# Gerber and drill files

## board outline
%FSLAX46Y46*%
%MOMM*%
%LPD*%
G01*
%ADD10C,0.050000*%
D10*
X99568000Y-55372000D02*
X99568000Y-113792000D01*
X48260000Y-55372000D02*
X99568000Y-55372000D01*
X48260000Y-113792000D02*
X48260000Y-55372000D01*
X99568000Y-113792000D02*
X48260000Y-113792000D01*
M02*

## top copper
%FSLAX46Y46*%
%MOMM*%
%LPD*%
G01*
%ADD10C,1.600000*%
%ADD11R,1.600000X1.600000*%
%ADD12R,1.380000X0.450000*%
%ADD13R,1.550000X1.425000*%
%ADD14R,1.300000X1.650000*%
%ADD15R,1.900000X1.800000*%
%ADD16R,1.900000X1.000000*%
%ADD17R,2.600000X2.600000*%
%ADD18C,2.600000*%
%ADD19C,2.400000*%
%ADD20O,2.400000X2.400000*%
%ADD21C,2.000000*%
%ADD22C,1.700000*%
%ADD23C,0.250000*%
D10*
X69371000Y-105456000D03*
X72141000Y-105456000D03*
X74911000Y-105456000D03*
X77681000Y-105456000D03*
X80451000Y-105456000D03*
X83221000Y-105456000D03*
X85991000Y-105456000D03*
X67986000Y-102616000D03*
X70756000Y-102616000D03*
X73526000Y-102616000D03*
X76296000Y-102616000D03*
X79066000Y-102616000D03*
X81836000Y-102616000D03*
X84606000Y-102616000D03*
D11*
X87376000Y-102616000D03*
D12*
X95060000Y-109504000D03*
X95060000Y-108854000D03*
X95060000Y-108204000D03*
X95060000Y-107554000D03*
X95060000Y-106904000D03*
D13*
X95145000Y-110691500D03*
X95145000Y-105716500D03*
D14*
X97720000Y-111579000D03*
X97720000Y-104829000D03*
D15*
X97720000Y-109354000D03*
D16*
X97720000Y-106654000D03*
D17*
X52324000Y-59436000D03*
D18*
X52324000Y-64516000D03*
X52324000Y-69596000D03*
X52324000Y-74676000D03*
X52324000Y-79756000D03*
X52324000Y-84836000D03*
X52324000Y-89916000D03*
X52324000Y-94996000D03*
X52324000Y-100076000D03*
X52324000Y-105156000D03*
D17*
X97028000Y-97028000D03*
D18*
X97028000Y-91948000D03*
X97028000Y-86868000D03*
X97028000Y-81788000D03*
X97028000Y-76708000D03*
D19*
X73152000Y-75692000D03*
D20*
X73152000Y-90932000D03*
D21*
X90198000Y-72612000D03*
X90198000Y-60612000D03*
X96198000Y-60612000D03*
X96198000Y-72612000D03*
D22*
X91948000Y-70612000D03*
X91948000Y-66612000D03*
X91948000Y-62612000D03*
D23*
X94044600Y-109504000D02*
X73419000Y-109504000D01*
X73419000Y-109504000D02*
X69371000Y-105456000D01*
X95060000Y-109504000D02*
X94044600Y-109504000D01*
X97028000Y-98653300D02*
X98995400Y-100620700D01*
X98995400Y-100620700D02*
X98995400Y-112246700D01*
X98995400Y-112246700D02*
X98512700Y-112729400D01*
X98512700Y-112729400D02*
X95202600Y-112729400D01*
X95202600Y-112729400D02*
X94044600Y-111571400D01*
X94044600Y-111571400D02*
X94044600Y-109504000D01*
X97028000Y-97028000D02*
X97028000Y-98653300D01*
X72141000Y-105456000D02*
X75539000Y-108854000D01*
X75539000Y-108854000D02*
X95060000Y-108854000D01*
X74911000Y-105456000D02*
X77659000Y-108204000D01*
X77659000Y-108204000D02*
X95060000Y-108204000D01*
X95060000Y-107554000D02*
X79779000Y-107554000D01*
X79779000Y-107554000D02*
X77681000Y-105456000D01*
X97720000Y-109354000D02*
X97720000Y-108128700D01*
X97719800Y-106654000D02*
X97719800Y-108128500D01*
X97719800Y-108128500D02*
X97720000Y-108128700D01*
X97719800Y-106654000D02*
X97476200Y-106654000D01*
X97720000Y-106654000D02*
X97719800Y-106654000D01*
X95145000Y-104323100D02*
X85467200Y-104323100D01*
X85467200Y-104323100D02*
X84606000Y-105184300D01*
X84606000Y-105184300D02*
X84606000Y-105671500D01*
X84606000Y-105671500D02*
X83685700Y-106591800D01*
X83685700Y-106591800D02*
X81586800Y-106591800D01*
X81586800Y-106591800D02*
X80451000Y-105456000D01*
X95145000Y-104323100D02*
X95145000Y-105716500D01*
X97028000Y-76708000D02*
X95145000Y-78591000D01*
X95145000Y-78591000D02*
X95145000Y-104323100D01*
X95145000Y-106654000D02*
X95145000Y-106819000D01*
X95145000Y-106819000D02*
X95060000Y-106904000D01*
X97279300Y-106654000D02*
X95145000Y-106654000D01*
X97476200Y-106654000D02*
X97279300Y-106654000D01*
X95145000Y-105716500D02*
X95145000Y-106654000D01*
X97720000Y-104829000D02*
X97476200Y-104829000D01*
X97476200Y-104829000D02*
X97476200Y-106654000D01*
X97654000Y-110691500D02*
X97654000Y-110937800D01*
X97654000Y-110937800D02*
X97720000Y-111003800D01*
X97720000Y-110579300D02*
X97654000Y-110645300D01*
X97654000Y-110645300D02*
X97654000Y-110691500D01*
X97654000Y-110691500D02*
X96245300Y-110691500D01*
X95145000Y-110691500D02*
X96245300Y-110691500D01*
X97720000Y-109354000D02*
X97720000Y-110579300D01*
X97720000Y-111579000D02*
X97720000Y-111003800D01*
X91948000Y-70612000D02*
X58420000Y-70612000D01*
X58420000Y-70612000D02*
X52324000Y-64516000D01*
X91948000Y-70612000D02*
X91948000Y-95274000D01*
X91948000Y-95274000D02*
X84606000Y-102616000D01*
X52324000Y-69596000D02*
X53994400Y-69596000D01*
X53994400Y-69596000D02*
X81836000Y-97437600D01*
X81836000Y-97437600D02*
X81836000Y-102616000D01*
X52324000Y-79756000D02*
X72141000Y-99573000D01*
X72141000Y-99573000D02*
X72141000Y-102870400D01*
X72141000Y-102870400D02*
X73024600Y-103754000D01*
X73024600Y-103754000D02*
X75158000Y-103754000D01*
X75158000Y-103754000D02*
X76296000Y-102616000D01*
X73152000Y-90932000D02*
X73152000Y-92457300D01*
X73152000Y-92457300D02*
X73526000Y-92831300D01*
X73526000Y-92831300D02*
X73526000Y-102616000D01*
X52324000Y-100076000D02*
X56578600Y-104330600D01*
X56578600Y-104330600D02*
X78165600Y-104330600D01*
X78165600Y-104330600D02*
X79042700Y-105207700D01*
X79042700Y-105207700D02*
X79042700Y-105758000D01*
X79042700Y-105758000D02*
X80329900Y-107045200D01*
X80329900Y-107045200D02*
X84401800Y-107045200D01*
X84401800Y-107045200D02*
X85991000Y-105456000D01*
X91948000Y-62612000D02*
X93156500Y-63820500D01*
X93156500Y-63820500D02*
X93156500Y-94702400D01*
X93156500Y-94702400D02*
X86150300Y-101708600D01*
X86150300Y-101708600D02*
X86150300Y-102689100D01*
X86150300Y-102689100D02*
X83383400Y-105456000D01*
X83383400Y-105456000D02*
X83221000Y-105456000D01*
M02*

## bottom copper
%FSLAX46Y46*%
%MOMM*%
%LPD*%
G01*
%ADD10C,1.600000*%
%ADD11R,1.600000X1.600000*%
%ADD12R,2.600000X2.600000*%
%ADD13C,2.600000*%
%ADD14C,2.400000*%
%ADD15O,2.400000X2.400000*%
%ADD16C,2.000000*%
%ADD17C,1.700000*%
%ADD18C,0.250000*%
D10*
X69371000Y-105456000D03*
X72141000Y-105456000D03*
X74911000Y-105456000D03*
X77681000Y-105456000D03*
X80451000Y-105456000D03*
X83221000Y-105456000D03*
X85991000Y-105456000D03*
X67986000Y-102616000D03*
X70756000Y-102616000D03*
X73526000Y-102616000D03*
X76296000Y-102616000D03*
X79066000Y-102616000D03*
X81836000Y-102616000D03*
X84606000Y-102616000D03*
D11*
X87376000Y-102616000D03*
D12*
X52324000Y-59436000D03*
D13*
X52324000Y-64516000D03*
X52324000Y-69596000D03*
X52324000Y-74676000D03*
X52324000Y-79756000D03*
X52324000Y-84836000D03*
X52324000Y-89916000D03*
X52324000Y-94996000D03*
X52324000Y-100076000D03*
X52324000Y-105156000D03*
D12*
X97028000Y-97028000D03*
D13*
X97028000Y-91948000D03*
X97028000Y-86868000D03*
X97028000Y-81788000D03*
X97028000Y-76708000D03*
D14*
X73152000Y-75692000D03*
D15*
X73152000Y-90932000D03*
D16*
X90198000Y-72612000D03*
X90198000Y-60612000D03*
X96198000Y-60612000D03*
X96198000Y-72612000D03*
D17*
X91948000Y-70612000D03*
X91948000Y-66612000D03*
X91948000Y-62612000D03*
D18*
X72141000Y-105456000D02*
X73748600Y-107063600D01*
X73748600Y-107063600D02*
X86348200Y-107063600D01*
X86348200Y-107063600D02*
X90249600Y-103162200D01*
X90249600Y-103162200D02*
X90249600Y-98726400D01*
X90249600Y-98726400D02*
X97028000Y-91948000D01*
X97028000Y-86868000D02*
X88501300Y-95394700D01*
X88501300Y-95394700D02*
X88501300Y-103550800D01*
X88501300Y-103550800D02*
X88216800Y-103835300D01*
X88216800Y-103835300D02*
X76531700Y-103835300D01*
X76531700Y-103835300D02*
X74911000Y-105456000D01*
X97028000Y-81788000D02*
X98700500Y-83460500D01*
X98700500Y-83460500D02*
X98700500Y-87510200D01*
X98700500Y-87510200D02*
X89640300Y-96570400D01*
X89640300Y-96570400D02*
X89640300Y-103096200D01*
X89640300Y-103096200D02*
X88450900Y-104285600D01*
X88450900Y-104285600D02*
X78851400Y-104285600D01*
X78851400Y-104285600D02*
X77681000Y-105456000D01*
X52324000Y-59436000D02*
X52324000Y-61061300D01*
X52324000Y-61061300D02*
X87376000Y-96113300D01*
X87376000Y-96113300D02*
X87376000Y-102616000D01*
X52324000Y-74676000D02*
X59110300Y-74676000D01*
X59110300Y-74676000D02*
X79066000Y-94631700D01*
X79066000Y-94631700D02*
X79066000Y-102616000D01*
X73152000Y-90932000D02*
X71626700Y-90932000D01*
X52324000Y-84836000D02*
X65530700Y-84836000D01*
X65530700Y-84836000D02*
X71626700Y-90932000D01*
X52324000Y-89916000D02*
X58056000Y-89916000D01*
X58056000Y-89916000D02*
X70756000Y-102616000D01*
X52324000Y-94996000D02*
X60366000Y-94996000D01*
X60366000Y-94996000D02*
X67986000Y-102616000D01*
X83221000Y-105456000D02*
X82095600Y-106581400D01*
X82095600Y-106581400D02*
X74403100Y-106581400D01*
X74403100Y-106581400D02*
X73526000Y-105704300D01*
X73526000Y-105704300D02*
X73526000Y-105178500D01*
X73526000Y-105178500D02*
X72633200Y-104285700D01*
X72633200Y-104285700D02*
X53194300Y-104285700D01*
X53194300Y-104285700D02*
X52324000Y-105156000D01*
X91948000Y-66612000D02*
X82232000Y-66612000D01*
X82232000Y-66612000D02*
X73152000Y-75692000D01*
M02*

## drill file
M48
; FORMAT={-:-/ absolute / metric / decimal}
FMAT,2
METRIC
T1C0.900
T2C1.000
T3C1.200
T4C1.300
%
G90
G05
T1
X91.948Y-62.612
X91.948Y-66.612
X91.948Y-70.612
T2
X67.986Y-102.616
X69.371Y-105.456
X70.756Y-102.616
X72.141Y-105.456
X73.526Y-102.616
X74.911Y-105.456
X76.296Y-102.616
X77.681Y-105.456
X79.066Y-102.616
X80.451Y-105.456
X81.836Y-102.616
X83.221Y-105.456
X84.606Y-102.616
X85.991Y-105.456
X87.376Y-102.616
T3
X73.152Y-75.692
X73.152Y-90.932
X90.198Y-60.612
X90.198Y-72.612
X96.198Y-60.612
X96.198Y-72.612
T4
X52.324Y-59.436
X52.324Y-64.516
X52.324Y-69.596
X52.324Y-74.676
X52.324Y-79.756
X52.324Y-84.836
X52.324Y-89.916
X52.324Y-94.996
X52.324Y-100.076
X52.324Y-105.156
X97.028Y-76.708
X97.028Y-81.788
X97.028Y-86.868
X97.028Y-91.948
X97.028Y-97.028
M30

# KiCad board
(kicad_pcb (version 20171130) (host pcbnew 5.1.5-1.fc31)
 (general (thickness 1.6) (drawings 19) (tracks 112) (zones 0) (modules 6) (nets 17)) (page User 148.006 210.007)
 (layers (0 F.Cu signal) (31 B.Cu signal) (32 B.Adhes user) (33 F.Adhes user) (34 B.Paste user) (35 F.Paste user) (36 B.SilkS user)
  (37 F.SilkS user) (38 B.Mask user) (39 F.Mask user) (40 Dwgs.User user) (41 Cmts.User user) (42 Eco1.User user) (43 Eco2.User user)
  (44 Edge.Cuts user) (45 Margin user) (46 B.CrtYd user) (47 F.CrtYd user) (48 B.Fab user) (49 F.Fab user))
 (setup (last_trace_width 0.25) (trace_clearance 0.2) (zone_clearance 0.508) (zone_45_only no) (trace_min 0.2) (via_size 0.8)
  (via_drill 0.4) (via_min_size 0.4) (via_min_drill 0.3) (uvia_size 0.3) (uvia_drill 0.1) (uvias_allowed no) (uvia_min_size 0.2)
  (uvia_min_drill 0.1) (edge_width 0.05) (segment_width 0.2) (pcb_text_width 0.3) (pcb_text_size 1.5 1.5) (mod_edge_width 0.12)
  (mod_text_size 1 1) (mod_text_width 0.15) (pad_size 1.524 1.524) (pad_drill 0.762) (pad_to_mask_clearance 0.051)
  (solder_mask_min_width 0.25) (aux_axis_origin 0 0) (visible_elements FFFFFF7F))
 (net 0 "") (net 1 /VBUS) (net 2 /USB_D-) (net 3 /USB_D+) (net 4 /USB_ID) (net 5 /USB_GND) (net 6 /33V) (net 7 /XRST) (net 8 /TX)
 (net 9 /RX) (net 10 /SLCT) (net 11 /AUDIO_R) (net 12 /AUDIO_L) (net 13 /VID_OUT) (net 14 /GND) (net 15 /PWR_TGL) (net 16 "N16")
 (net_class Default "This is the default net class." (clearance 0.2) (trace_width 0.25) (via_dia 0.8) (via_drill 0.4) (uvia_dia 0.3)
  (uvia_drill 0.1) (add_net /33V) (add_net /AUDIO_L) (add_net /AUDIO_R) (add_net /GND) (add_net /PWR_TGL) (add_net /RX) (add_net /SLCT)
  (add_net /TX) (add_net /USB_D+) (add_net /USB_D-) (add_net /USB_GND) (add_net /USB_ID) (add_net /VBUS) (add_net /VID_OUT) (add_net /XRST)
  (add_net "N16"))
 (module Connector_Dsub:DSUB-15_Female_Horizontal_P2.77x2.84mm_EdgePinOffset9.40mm (layer F.Cu) (at 87.376 102.616)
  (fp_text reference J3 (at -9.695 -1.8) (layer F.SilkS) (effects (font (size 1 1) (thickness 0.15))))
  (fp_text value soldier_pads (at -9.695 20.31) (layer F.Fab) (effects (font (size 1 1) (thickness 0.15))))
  (pad 15 thru_hole circle (at -18.005 2.84) (size 1.6 1.6) (drill 1) (layers *.Cu *.Mask) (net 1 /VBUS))
  (pad 14 thru_hole circle (at -15.235 2.84) (size 1.6 1.6) (drill 1) (layers *.Cu *.Mask) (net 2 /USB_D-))
  (pad 13 thru_hole circle (at -12.465 2.84) (size 1.6 1.6) (drill 1) (layers *.Cu *.Mask) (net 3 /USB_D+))
  (pad 12 thru_hole circle (at -9.695 2.84) (size 1.6 1.6) (drill 1) (layers *.Cu *.Mask) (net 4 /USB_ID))
  (pad 11 thru_hole circle (at -6.925 2.84) (size 1.6 1.6) (drill 1) (layers *.Cu *.Mask) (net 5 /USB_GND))
  (pad 10 thru_hole circle (at -4.155 2.84) (size 1.6 1.6) (drill 1) (layers *.Cu *.Mask) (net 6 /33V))
  (pad 9 thru_hole circle (at -1.385 2.84) (size 1.6 1.6) (drill 1) (layers *.Cu *.Mask) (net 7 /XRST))
  (pad 8 thru_hole circle (at -19.39 0) (size 1.6 1.6) (drill 1) (layers *.Cu *.Mask) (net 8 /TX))
  (pad 7 thru_hole circle (at -16.62 0) (size 1.6 1.6) (drill 1) (layers *.Cu *.Mask) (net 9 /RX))
  (pad 6 thru_hole circle (at -13.85 0) (size 1.6 1.6) (drill 1) (layers *.Cu *.Mask) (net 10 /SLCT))
  (pad 5 thru_hole circle (at -11.08 0) (size 1.6 1.6) (drill 1) (layers *.Cu *.Mask) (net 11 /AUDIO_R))
  (pad 4 thru_hole circle (at -8.31 0) (size 1.6 1.6) (drill 1) (layers *.Cu *.Mask) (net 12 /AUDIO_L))
  (pad 3 thru_hole circle (at -5.54 0) (size 1.6 1.6) (drill 1) (layers *.Cu *.Mask) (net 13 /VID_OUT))
  (pad 2 thru_hole circle (at -2.77 0) (size 1.6 1.6) (drill 1) (layers *.Cu *.Mask) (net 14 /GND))
  (pad 1 thru_hole rect (at 0 0) (size 1.6 1.6) (drill 1) (layers *.Cu *.Mask) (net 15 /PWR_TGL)))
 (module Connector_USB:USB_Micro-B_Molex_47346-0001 (layer F.Cu) (at 96.52 108.204 90)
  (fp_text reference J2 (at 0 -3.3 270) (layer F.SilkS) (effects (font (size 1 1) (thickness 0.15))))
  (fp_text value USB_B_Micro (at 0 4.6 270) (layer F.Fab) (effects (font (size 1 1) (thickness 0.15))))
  (pad 1 smd rect (at -1.3 -1.46 90) (size 0.45 1.38) (layers F.Cu F.Paste F.Mask) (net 1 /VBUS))
  (pad 2 smd rect (at -0.65 -1.46 90) (size 0.45 1.38) (layers F.Cu F.Paste F.Mask) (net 2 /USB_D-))
  (pad 3 smd rect (at 0 -1.46 90) (size 0.45 1.38) (layers F.Cu F.Paste F.Mask) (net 3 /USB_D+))
  (pad 4 smd rect (at 0.65 -1.46 90) (size 0.45 1.38) (layers F.Cu F.Paste F.Mask) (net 4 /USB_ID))
  (pad 5 smd rect (at 1.3 -1.46 90) (size 0.45 1.38) (layers F.Cu F.Paste F.Mask) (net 5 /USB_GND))
  (pad 6 smd rect (at -2.4875 -1.375 90) (size 1.425 1.55) (layers F.Cu F.Paste F.Mask) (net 5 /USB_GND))
  (pad 6 smd rect (at 2.4875 -1.375 90) (size 1.425 1.55) (layers F.Cu F.Paste F.Mask) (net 5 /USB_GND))
  (pad 6 smd rect (at -3.375 1.2 90) (size 1.65 1.3) (layers F.Cu F.Paste F.Mask) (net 5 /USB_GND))
  (pad 6 smd rect (at 3.375 1.2 90) (size 1.65 1.3) (layers F.Cu F.Paste F.Mask) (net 5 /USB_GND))
  (pad 6 smd rect (at -1.15 1.2 90) (size 1.8 1.9) (layers F.Cu F.Paste F.Mask) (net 5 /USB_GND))
  (pad 6 smd rect (at 1.55 1.2 90) (size 1 1.9) (layers F.Cu F.Paste F.Mask) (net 5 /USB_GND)))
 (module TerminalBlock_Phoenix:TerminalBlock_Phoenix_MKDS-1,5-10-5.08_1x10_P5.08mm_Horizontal (layer F.Cu) (at 52.324 59.436 270)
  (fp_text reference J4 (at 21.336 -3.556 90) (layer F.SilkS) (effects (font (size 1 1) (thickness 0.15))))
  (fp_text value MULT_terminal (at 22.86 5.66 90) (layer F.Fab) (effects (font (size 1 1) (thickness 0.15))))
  (pad 1 thru_hole rect (at 0 0 270) (size 2.6 2.6) (drill 1.3) (layers *.Cu *.Mask) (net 15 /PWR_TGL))
  (pad 2 thru_hole circle (at 5.08 0 270) (size 2.6 2.6) (drill 1.3) (layers *.Cu *.Mask) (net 14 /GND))
  (pad 3 thru_hole circle (at 10.16 0 270) (size 2.6 2.6) (drill 1.3) (layers *.Cu *.Mask) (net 13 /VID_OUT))
  (pad 4 thru_hole circle (at 15.24 0 270) (size 2.6 2.6) (drill 1.3) (layers *.Cu *.Mask) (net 12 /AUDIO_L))
  (pad 5 thru_hole circle (at 20.32 0 270) (size 2.6 2.6) (drill 1.3) (layers *.Cu *.Mask) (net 11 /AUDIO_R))
  (pad 6 thru_hole circle (at 25.4 0 270) (size 2.6 2.6) (drill 1.3) (layers *.Cu *.Mask) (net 10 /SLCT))
  (pad 7 thru_hole circle (at 30.48 0 270) (size 2.6 2.6) (drill 1.3) (layers *.Cu *.Mask) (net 9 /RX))
  (pad 8 thru_hole circle (at 35.56 0 270) (size 2.6 2.6) (drill 1.3) (layers *.Cu *.Mask) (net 8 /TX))
  (pad 9 thru_hole circle (at 40.64 0 270) (size 2.6 2.6) (drill 1.3) (layers *.Cu *.Mask) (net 7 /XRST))
  (pad 10 thru_hole circle (at 45.72 0 270) (size 2.6 2.6) (drill 1.3) (layers *.Cu *.Mask) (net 6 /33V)))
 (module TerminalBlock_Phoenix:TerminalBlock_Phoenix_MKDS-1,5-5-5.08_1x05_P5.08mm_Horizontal (layer F.Cu) (at 97.028 97.028 90)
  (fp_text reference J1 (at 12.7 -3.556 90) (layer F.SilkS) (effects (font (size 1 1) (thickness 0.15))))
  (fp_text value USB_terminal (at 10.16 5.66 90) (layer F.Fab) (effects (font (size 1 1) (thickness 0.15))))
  (pad 1 thru_hole rect (at 0 0 90) (size 2.6 2.6) (drill 1.3) (layers *.Cu *.Mask) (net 1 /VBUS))
  (pad 2 thru_hole circle (at 5.08 0 90) (size 2.6 2.6) (drill 1.3) (layers *.Cu *.Mask) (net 2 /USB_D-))
  (pad 3 thru_hole circle (at 10.16 0 90) (size 2.6 2.6) (drill 1.3) (layers *.Cu *.Mask) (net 3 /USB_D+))
  (pad 4 thru_hole circle (at 15.24 0 90) (size 2.6 2.6) (drill 1.3) (layers *.Cu *.Mask) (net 4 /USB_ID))
  (pad 5 thru_hole circle (at 20.32 0 90) (size 2.6 2.6) (drill 1.3) (layers *.Cu *.Mask) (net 5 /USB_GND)))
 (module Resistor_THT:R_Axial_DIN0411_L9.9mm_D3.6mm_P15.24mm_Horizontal (layer F.Cu) (at 73.152 75.692 270)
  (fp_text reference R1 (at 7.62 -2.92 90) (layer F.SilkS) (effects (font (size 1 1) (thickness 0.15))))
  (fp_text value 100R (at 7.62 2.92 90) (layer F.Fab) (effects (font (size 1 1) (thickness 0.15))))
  (pad 1 thru_hole circle (at 0 0 270) (size 2.4 2.4) (drill 1.2) (layers *.Cu *.Mask) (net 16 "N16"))
  (pad 2 thru_hole oval (at 15.24 0 270) (size 2.4 2.4) (drill 1.2) (layers *.Cu *.Mask) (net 10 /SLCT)))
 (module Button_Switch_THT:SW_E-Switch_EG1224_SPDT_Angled (layer F.Cu) (at 91.948 70.612 90)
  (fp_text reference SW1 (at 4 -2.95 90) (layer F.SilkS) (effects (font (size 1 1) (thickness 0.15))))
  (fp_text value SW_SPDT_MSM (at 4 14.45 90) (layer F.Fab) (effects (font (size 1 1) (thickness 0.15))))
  (pad "" thru_hole circle (at -2 -1.75 90) (size 2 2) (drill 1.2) (layers *.Cu *.Mask))
  (pad "" thru_hole circle (at 10 -1.75 90) (size 2 2) (drill 1.2) (layers *.Cu *.Mask))
  (pad "" thru_hole circle (at 10 4.25 90) (size 2 2) (drill 1.2) (layers *.Cu *.Mask))
  (pad "" thru_hole circle (at -2 4.25 90) (size 2 2) (drill 1.2) (layers *.Cu *.Mask))
  (pad 1 thru_hole circle (at 0 0 90) (size 1.7 1.7) (drill 0.9) (layers *.Cu *.Mask) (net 14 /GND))
  (pad 2 thru_hole circle (at 4 0 90) (size 1.7 1.7) (drill 0.9) (layers *.Cu *.Mask) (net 16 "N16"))
  (pad 3 thru_hole circle (at 8 0 90) (size 1.7 1.7) (drill 0.9) (layers *.Cu *.Mask) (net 6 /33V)))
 (gr_line (start 99.568 55.372) (end 99.568 113.792) (layer Edge.Cuts) (width 0.05))
 (gr_line (start 48.26 55.372) (end 99.568 55.372) (layer Edge.Cuts) (width 0.05))
 (gr_line (start 48.26 113.792) (end 48.26 55.372) (layer Edge.Cuts) (width 0.05))
 (gr_line (start 99.568 113.792) (end 48.26 113.792) (layer Edge.Cuts) (width 0.05))
 (segment (start 94.0446 109.504) (end 73.419 109.504) (width 0.25) (layer F.Cu) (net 1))
 (segment (start 73.419 109.504) (end 69.371 105.456) (width 0.25) (layer F.Cu) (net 1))
 (segment (start 95.06 109.504) (end 94.0446 109.504) (width 0.25) (layer F.Cu) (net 1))
 (segment (start 97.028 98.6533) (end 98.9954 100.6207) (width 0.25) (layer F.Cu) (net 1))
 (segment (start 98.9954 100.6207) (end 98.9954 112.2467) (width 0.25) (layer F.Cu) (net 1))
 (segment (start 98.9954 112.2467) (end 98.5127 112.7294) (width 0.25) (layer F.Cu) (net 1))
 (segment (start 98.5127 112.7294) (end 95.2026 112.7294) (width 0.25) (layer F.Cu) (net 1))
 (segment (start 95.2026 112.7294) (end 94.0446 111.5714) (width 0.25) (layer F.Cu) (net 1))
 (segment (start 94.0446 111.5714) (end 94.0446 109.504) (width 0.25) (layer F.Cu) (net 1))
 (segment (start 97.028 97.028) (end 97.028 98.6533) (width 0.25) (layer F.Cu) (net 1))
 (segment (start 72.141 105.456) (end 73.7486 107.0636) (width 0.25) (layer B.Cu) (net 2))
 (segment (start 73.7486 107.0636) (end 86.3482 107.0636) (width 0.25) (layer B.Cu) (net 2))
 (segment (start 86.3482 107.0636) (end 90.2496 103.1622) (width 0.25) (layer B.Cu) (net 2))
 (segment (start 90.2496 103.1622) (end 90.2496 98.7264) (width 0.25) (layer B.Cu) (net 2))
 (segment (start 90.2496 98.7264) (end 97.028 91.948) (width 0.25) (layer B.Cu) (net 2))
 (segment (start 72.141 105.456) (end 75.539 108.854) (width 0.25) (layer F.Cu) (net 2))
 (segment (start 75.539 108.854) (end 95.06 108.854) (width 0.25) (layer F.Cu) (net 2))
 (segment (start 97.028 86.868) (end 88.5013 95.3947) (width 0.25) (layer B.Cu) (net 3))
 (segment (start 88.5013 95.3947) (end 88.5013 103.5508) (width 0.25) (layer B.Cu) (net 3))
 (segment (start 88.5013 103.5508) (end 88.2168 103.8353) (width 0.25) (layer B.Cu) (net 3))
 (segment (start 88.2168 103.8353) (end 76.5317 103.8353) (width 0.25) (layer B.Cu) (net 3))
 (segment (start 76.5317 103.8353) (end 74.911 105.456) (width 0.25) (layer B.Cu) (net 3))
 (segment (start 74.911 105.456) (end 77.659 108.204) (width 0.25) (layer F.Cu) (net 3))
 (segment (start 77.659 108.204) (end 95.06 108.204) (width 0.25) (layer F.Cu) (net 3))
 (segment (start 97.028 81.788) (end 98.7005 83.4605) (width 0.25) (layer B.Cu) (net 4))
 (segment (start 98.7005 83.4605) (end 98.7005 87.5102) (width 0.25) (layer B.Cu) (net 4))
 (segment (start 98.7005 87.5102) (end 89.6403 96.5704) (width 0.25) (layer B.Cu) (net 4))
 (segment (start 89.6403 96.5704) (end 89.6403 103.0962) (width 0.25) (layer B.Cu) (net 4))
 (segment (start 89.6403 103.0962) (end 88.4509 104.2856) (width 0.25) (layer B.Cu) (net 4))
 (segment (start 88.4509 104.2856) (end 78.8514 104.2856) (width 0.25) (layer B.Cu) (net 4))
 (segment (start 78.8514 104.2856) (end 77.681 105.456) (width 0.25) (layer B.Cu) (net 4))
 (segment (start 95.06 107.554) (end 79.779 107.554) (width 0.25) (layer F.Cu) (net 4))
 (segment (start 79.779 107.554) (end 77.681 105.456) (width 0.25) (layer F.Cu) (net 4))
 (segment (start 97.72 109.354) (end 97.72 108.1287) (width 0.25) (layer F.Cu) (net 5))
 (segment (start 97.7198 106.654) (end 97.7198 108.1285) (width 0.25) (layer F.Cu) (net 5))
 (segment (start 97.7198 108.1285) (end 97.72 108.1287) (width 0.25) (layer F.Cu) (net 5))
 (segment (start 97.7198 106.654) (end 97.4762 106.654) (width 0.25) (layer F.Cu) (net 5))
 (segment (start 97.72 106.654) (end 97.7198 106.654) (width 0.25) (layer F.Cu) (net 5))
 (segment (start 95.145 104.3231) (end 85.4672 104.3231) (width 0.25) (layer F.Cu) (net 5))
 (segment (start 85.4672 104.3231) (end 84.606 105.1843) (width 0.25) (layer F.Cu) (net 5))
 (segment (start 84.606 105.1843) (end 84.606 105.6715) (width 0.25) (layer F.Cu) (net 5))
 (segment (start 84.606 105.6715) (end 83.6857 106.5918) (width 0.25) (layer F.Cu) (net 5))
 (segment (start 83.6857 106.5918) (end 81.5868 106.5918) (width 0.25) (layer F.Cu) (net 5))
 (segment (start 81.5868 106.5918) (end 80.451 105.456) (width 0.25) (layer F.Cu) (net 5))
 (segment (start 95.145 104.3231) (end 95.145 105.7165) (width 0.25) (layer F.Cu) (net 5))
 (segment (start 97.028 76.708) (end 95.145 78.591) (width 0.25) (layer F.Cu) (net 5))
 (segment (start 95.145 78.591) (end 95.145 104.3231) (width 0.25) (layer F.Cu) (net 5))
 (segment (start 95.145 106.654) (end 95.145 106.819) (width 0.25) (layer F.Cu) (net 5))
 (segment (start 95.145 106.819) (end 95.06 106.904) (width 0.25) (layer F.Cu) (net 5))
 (segment (start 97.2793 106.654) (end 95.145 106.654) (width 0.25) (layer F.Cu) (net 5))
 (segment (start 97.4762 106.654) (end 97.2793 106.654) (width 0.25) (layer F.Cu) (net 5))
 (segment (start 95.145 105.7165) (end 95.145 106.654) (width 0.25) (layer F.Cu) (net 5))
 (segment (start 97.72 104.829) (end 97.4762 104.829) (width 0.25) (layer F.Cu) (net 5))
 (segment (start 97.4762 104.829) (end 97.4762 106.654) (width 0.25) (layer F.Cu) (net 5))
 (segment (start 97.654 110.6915) (end 97.654 110.9378) (width 0.25) (layer F.Cu) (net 5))
 (segment (start 97.654 110.9378) (end 97.72 111.0038) (width 0.25) (layer F.Cu) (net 5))
 (segment (start 97.72 110.5793) (end 97.654 110.6453) (width 0.25) (layer F.Cu) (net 5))
 (segment (start 97.654 110.6453) (end 97.654 110.6915) (width 0.25) (layer F.Cu) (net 5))
 (segment (start 97.654 110.6915) (end 96.2453 110.6915) (width 0.25) (layer F.Cu) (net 5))
 (segment (start 95.145 110.6915) (end 96.2453 110.6915) (width 0.25) (layer F.Cu) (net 5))
 (segment (start 97.72 109.354) (end 97.72 110.5793) (width 0.25) (layer F.Cu) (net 5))
 (segment (start 97.72 111.579) (end 97.72 111.0038) (width 0.25) (layer F.Cu) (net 5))
 (segment (start 52.324 59.436) (end 52.324 61.0613) (width 0.25) (layer B.Cu) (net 15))
 (segment (start 52.324 61.0613) (end 87.376 96.1133) (width 0.25) (layer B.Cu) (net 15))
 (segment (start 87.376 96.1133) (end 87.376 102.616) (width 0.25) (layer B.Cu) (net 15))
 (segment (start 91.948 70.612) (end 58.42 70.612) (width 0.25) (layer F.Cu) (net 14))
 (segment (start 58.42 70.612) (end 52.324 64.516) (width 0.25) (layer F.Cu) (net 14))
 (segment (start 91.948 70.612) (end 91.948 95.274) (width 0.25) (layer F.Cu) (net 14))
 (segment (start 91.948 95.274) (end 84.606 102.616) (width 0.25) (layer F.Cu) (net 14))
 (segment (start 52.324 69.596) (end 53.9944 69.596) (width 0.25) (layer F.Cu) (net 13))
 (segment (start 53.9944 69.596) (end 81.836 97.4376) (width 0.25) (layer F.Cu) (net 13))
 (segment (start 81.836 97.4376) (end 81.836 102.616) (width 0.25) (layer F.Cu) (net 13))
 (segment (start 52.324 74.676) (end 59.1103 74.676) (width 0.25) (layer B.Cu) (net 12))
 (segment (start 59.1103 74.676) (end 79.066 94.6317) (width 0.25) (layer B.Cu) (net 12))
 (segment (start 79.066 94.6317) (end 79.066 102.616) (width 0.25) (layer B.Cu) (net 12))
 (segment (start 52.324 79.756) (end 72.141 99.573) (width 0.25) (layer F.Cu) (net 11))
 (segment (start 72.141 99.573) (end 72.141 102.8704) (width 0.25) (layer F.Cu) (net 11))
 (segment (start 72.141 102.8704) (end 73.0246 103.754) (width 0.25) (layer F.Cu) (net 11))
 (segment (start 73.0246 103.754) (end 75.158 103.754) (width 0.25) (layer F.Cu) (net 11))
 (segment (start 75.158 103.754) (end 76.296 102.616) (width 0.25) (layer F.Cu) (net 11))
 (segment (start 73.152 90.932) (end 71.6267 90.932) (width 0.25) (layer B.Cu) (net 10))
 (segment (start 52.324 84.836) (end 65.5307 84.836) (width 0.25) (layer B.Cu) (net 10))
 (segment (start 65.5307 84.836) (end 71.6267 90.932) (width 0.25) (layer B.Cu) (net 10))
 (segment (start 73.152 90.932) (end 73.152 92.4573) (width 0.25) (layer F.Cu) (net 10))
 (segment (start 73.152 92.4573) (end 73.526 92.8313) (width 0.25) (layer F.Cu) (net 10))
 (segment (start 73.526 92.8313) (end 73.526 102.616) (width 0.25) (layer F.Cu) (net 10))
 (segment (start 52.324 89.916) (end 58.056 89.916) (width 0.25) (layer B.Cu) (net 9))
 (segment (start 58.056 89.916) (end 70.756 102.616) (width 0.25) (layer B.Cu) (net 9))
 (segment (start 52.324 94.996) (end 60.366 94.996) (width 0.25) (layer B.Cu) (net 8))
 (segment (start 60.366 94.996) (end 67.986 102.616) (width 0.25) (layer B.Cu) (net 8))
 (segment (start 52.324 100.076) (end 56.5786 104.3306) (width 0.25) (layer F.Cu) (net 7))
 (segment (start 56.5786 104.3306) (end 78.1656 104.3306) (width 0.25) (layer F.Cu) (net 7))
 (segment (start 78.1656 104.3306) (end 79.0427 105.2077) (width 0.25) (layer F.Cu) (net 7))
 (segment (start 79.0427 105.2077) (end 79.0427 105.758) (width 0.25) (layer F.Cu) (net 7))
 (segment (start 79.0427 105.758) (end 80.3299 107.0452) (width 0.25) (layer F.Cu) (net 7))
 (segment (start 80.3299 107.0452) (end 84.4018 107.0452) (width 0.25) (layer F.Cu) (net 7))
 (segment (start 84.4018 107.0452) (end 85.991 105.456) (width 0.25) (layer F.Cu) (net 7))
 (segment (start 83.221 105.456) (end 82.0956 106.5814) (width 0.25) (layer B.Cu) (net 6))
 (segment (start 82.0956 106.5814) (end 74.4031 106.5814) (width 0.25) (layer B.Cu) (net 6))
 (segment (start 74.4031 106.5814) (end 73.526 105.7043) (width 0.25) (layer B.Cu) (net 6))
 (segment (start 73.526 105.7043) (end 73.526 105.1785) (width 0.25) (layer B.Cu) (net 6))
 (segment (start 73.526 105.1785) (end 72.6332 104.2857) (width 0.25) (layer B.Cu) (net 6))
 (segment (start 72.6332 104.2857) (end 53.1943 104.2857) (width 0.25) (layer B.Cu) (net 6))
 (segment (start 53.1943 104.2857) (end 52.324 105.156) (width 0.25) (layer B.Cu) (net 6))
 (segment (start 91.948 62.612) (end 93.1565 63.8205) (width 0.25) (layer F.Cu) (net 6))
 (segment (start 93.1565 63.8205) (end 93.1565 94.7024) (width 0.25) (layer F.Cu) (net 6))
 (segment (start 93.1565 94.7024) (end 86.1503 101.7086) (width 0.25) (layer F.Cu) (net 6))
 (segment (start 86.1503 101.7086) (end 86.1503 102.6891) (width 0.25) (layer F.Cu) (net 6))
 (segment (start 86.1503 102.6891) (end 83.3834 105.456) (width 0.25) (layer F.Cu) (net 6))
 (segment (start 83.3834 105.456) (end 83.221 105.456) (width 0.25) (layer F.Cu) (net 6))
 (segment (start 91.948 66.612) (end 82.232 66.612) (width 0.25) (layer B.Cu) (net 16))
 (segment (start 82.232 66.612) (end 73.152 75.692) (width 0.25) (layer B.Cu) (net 16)))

